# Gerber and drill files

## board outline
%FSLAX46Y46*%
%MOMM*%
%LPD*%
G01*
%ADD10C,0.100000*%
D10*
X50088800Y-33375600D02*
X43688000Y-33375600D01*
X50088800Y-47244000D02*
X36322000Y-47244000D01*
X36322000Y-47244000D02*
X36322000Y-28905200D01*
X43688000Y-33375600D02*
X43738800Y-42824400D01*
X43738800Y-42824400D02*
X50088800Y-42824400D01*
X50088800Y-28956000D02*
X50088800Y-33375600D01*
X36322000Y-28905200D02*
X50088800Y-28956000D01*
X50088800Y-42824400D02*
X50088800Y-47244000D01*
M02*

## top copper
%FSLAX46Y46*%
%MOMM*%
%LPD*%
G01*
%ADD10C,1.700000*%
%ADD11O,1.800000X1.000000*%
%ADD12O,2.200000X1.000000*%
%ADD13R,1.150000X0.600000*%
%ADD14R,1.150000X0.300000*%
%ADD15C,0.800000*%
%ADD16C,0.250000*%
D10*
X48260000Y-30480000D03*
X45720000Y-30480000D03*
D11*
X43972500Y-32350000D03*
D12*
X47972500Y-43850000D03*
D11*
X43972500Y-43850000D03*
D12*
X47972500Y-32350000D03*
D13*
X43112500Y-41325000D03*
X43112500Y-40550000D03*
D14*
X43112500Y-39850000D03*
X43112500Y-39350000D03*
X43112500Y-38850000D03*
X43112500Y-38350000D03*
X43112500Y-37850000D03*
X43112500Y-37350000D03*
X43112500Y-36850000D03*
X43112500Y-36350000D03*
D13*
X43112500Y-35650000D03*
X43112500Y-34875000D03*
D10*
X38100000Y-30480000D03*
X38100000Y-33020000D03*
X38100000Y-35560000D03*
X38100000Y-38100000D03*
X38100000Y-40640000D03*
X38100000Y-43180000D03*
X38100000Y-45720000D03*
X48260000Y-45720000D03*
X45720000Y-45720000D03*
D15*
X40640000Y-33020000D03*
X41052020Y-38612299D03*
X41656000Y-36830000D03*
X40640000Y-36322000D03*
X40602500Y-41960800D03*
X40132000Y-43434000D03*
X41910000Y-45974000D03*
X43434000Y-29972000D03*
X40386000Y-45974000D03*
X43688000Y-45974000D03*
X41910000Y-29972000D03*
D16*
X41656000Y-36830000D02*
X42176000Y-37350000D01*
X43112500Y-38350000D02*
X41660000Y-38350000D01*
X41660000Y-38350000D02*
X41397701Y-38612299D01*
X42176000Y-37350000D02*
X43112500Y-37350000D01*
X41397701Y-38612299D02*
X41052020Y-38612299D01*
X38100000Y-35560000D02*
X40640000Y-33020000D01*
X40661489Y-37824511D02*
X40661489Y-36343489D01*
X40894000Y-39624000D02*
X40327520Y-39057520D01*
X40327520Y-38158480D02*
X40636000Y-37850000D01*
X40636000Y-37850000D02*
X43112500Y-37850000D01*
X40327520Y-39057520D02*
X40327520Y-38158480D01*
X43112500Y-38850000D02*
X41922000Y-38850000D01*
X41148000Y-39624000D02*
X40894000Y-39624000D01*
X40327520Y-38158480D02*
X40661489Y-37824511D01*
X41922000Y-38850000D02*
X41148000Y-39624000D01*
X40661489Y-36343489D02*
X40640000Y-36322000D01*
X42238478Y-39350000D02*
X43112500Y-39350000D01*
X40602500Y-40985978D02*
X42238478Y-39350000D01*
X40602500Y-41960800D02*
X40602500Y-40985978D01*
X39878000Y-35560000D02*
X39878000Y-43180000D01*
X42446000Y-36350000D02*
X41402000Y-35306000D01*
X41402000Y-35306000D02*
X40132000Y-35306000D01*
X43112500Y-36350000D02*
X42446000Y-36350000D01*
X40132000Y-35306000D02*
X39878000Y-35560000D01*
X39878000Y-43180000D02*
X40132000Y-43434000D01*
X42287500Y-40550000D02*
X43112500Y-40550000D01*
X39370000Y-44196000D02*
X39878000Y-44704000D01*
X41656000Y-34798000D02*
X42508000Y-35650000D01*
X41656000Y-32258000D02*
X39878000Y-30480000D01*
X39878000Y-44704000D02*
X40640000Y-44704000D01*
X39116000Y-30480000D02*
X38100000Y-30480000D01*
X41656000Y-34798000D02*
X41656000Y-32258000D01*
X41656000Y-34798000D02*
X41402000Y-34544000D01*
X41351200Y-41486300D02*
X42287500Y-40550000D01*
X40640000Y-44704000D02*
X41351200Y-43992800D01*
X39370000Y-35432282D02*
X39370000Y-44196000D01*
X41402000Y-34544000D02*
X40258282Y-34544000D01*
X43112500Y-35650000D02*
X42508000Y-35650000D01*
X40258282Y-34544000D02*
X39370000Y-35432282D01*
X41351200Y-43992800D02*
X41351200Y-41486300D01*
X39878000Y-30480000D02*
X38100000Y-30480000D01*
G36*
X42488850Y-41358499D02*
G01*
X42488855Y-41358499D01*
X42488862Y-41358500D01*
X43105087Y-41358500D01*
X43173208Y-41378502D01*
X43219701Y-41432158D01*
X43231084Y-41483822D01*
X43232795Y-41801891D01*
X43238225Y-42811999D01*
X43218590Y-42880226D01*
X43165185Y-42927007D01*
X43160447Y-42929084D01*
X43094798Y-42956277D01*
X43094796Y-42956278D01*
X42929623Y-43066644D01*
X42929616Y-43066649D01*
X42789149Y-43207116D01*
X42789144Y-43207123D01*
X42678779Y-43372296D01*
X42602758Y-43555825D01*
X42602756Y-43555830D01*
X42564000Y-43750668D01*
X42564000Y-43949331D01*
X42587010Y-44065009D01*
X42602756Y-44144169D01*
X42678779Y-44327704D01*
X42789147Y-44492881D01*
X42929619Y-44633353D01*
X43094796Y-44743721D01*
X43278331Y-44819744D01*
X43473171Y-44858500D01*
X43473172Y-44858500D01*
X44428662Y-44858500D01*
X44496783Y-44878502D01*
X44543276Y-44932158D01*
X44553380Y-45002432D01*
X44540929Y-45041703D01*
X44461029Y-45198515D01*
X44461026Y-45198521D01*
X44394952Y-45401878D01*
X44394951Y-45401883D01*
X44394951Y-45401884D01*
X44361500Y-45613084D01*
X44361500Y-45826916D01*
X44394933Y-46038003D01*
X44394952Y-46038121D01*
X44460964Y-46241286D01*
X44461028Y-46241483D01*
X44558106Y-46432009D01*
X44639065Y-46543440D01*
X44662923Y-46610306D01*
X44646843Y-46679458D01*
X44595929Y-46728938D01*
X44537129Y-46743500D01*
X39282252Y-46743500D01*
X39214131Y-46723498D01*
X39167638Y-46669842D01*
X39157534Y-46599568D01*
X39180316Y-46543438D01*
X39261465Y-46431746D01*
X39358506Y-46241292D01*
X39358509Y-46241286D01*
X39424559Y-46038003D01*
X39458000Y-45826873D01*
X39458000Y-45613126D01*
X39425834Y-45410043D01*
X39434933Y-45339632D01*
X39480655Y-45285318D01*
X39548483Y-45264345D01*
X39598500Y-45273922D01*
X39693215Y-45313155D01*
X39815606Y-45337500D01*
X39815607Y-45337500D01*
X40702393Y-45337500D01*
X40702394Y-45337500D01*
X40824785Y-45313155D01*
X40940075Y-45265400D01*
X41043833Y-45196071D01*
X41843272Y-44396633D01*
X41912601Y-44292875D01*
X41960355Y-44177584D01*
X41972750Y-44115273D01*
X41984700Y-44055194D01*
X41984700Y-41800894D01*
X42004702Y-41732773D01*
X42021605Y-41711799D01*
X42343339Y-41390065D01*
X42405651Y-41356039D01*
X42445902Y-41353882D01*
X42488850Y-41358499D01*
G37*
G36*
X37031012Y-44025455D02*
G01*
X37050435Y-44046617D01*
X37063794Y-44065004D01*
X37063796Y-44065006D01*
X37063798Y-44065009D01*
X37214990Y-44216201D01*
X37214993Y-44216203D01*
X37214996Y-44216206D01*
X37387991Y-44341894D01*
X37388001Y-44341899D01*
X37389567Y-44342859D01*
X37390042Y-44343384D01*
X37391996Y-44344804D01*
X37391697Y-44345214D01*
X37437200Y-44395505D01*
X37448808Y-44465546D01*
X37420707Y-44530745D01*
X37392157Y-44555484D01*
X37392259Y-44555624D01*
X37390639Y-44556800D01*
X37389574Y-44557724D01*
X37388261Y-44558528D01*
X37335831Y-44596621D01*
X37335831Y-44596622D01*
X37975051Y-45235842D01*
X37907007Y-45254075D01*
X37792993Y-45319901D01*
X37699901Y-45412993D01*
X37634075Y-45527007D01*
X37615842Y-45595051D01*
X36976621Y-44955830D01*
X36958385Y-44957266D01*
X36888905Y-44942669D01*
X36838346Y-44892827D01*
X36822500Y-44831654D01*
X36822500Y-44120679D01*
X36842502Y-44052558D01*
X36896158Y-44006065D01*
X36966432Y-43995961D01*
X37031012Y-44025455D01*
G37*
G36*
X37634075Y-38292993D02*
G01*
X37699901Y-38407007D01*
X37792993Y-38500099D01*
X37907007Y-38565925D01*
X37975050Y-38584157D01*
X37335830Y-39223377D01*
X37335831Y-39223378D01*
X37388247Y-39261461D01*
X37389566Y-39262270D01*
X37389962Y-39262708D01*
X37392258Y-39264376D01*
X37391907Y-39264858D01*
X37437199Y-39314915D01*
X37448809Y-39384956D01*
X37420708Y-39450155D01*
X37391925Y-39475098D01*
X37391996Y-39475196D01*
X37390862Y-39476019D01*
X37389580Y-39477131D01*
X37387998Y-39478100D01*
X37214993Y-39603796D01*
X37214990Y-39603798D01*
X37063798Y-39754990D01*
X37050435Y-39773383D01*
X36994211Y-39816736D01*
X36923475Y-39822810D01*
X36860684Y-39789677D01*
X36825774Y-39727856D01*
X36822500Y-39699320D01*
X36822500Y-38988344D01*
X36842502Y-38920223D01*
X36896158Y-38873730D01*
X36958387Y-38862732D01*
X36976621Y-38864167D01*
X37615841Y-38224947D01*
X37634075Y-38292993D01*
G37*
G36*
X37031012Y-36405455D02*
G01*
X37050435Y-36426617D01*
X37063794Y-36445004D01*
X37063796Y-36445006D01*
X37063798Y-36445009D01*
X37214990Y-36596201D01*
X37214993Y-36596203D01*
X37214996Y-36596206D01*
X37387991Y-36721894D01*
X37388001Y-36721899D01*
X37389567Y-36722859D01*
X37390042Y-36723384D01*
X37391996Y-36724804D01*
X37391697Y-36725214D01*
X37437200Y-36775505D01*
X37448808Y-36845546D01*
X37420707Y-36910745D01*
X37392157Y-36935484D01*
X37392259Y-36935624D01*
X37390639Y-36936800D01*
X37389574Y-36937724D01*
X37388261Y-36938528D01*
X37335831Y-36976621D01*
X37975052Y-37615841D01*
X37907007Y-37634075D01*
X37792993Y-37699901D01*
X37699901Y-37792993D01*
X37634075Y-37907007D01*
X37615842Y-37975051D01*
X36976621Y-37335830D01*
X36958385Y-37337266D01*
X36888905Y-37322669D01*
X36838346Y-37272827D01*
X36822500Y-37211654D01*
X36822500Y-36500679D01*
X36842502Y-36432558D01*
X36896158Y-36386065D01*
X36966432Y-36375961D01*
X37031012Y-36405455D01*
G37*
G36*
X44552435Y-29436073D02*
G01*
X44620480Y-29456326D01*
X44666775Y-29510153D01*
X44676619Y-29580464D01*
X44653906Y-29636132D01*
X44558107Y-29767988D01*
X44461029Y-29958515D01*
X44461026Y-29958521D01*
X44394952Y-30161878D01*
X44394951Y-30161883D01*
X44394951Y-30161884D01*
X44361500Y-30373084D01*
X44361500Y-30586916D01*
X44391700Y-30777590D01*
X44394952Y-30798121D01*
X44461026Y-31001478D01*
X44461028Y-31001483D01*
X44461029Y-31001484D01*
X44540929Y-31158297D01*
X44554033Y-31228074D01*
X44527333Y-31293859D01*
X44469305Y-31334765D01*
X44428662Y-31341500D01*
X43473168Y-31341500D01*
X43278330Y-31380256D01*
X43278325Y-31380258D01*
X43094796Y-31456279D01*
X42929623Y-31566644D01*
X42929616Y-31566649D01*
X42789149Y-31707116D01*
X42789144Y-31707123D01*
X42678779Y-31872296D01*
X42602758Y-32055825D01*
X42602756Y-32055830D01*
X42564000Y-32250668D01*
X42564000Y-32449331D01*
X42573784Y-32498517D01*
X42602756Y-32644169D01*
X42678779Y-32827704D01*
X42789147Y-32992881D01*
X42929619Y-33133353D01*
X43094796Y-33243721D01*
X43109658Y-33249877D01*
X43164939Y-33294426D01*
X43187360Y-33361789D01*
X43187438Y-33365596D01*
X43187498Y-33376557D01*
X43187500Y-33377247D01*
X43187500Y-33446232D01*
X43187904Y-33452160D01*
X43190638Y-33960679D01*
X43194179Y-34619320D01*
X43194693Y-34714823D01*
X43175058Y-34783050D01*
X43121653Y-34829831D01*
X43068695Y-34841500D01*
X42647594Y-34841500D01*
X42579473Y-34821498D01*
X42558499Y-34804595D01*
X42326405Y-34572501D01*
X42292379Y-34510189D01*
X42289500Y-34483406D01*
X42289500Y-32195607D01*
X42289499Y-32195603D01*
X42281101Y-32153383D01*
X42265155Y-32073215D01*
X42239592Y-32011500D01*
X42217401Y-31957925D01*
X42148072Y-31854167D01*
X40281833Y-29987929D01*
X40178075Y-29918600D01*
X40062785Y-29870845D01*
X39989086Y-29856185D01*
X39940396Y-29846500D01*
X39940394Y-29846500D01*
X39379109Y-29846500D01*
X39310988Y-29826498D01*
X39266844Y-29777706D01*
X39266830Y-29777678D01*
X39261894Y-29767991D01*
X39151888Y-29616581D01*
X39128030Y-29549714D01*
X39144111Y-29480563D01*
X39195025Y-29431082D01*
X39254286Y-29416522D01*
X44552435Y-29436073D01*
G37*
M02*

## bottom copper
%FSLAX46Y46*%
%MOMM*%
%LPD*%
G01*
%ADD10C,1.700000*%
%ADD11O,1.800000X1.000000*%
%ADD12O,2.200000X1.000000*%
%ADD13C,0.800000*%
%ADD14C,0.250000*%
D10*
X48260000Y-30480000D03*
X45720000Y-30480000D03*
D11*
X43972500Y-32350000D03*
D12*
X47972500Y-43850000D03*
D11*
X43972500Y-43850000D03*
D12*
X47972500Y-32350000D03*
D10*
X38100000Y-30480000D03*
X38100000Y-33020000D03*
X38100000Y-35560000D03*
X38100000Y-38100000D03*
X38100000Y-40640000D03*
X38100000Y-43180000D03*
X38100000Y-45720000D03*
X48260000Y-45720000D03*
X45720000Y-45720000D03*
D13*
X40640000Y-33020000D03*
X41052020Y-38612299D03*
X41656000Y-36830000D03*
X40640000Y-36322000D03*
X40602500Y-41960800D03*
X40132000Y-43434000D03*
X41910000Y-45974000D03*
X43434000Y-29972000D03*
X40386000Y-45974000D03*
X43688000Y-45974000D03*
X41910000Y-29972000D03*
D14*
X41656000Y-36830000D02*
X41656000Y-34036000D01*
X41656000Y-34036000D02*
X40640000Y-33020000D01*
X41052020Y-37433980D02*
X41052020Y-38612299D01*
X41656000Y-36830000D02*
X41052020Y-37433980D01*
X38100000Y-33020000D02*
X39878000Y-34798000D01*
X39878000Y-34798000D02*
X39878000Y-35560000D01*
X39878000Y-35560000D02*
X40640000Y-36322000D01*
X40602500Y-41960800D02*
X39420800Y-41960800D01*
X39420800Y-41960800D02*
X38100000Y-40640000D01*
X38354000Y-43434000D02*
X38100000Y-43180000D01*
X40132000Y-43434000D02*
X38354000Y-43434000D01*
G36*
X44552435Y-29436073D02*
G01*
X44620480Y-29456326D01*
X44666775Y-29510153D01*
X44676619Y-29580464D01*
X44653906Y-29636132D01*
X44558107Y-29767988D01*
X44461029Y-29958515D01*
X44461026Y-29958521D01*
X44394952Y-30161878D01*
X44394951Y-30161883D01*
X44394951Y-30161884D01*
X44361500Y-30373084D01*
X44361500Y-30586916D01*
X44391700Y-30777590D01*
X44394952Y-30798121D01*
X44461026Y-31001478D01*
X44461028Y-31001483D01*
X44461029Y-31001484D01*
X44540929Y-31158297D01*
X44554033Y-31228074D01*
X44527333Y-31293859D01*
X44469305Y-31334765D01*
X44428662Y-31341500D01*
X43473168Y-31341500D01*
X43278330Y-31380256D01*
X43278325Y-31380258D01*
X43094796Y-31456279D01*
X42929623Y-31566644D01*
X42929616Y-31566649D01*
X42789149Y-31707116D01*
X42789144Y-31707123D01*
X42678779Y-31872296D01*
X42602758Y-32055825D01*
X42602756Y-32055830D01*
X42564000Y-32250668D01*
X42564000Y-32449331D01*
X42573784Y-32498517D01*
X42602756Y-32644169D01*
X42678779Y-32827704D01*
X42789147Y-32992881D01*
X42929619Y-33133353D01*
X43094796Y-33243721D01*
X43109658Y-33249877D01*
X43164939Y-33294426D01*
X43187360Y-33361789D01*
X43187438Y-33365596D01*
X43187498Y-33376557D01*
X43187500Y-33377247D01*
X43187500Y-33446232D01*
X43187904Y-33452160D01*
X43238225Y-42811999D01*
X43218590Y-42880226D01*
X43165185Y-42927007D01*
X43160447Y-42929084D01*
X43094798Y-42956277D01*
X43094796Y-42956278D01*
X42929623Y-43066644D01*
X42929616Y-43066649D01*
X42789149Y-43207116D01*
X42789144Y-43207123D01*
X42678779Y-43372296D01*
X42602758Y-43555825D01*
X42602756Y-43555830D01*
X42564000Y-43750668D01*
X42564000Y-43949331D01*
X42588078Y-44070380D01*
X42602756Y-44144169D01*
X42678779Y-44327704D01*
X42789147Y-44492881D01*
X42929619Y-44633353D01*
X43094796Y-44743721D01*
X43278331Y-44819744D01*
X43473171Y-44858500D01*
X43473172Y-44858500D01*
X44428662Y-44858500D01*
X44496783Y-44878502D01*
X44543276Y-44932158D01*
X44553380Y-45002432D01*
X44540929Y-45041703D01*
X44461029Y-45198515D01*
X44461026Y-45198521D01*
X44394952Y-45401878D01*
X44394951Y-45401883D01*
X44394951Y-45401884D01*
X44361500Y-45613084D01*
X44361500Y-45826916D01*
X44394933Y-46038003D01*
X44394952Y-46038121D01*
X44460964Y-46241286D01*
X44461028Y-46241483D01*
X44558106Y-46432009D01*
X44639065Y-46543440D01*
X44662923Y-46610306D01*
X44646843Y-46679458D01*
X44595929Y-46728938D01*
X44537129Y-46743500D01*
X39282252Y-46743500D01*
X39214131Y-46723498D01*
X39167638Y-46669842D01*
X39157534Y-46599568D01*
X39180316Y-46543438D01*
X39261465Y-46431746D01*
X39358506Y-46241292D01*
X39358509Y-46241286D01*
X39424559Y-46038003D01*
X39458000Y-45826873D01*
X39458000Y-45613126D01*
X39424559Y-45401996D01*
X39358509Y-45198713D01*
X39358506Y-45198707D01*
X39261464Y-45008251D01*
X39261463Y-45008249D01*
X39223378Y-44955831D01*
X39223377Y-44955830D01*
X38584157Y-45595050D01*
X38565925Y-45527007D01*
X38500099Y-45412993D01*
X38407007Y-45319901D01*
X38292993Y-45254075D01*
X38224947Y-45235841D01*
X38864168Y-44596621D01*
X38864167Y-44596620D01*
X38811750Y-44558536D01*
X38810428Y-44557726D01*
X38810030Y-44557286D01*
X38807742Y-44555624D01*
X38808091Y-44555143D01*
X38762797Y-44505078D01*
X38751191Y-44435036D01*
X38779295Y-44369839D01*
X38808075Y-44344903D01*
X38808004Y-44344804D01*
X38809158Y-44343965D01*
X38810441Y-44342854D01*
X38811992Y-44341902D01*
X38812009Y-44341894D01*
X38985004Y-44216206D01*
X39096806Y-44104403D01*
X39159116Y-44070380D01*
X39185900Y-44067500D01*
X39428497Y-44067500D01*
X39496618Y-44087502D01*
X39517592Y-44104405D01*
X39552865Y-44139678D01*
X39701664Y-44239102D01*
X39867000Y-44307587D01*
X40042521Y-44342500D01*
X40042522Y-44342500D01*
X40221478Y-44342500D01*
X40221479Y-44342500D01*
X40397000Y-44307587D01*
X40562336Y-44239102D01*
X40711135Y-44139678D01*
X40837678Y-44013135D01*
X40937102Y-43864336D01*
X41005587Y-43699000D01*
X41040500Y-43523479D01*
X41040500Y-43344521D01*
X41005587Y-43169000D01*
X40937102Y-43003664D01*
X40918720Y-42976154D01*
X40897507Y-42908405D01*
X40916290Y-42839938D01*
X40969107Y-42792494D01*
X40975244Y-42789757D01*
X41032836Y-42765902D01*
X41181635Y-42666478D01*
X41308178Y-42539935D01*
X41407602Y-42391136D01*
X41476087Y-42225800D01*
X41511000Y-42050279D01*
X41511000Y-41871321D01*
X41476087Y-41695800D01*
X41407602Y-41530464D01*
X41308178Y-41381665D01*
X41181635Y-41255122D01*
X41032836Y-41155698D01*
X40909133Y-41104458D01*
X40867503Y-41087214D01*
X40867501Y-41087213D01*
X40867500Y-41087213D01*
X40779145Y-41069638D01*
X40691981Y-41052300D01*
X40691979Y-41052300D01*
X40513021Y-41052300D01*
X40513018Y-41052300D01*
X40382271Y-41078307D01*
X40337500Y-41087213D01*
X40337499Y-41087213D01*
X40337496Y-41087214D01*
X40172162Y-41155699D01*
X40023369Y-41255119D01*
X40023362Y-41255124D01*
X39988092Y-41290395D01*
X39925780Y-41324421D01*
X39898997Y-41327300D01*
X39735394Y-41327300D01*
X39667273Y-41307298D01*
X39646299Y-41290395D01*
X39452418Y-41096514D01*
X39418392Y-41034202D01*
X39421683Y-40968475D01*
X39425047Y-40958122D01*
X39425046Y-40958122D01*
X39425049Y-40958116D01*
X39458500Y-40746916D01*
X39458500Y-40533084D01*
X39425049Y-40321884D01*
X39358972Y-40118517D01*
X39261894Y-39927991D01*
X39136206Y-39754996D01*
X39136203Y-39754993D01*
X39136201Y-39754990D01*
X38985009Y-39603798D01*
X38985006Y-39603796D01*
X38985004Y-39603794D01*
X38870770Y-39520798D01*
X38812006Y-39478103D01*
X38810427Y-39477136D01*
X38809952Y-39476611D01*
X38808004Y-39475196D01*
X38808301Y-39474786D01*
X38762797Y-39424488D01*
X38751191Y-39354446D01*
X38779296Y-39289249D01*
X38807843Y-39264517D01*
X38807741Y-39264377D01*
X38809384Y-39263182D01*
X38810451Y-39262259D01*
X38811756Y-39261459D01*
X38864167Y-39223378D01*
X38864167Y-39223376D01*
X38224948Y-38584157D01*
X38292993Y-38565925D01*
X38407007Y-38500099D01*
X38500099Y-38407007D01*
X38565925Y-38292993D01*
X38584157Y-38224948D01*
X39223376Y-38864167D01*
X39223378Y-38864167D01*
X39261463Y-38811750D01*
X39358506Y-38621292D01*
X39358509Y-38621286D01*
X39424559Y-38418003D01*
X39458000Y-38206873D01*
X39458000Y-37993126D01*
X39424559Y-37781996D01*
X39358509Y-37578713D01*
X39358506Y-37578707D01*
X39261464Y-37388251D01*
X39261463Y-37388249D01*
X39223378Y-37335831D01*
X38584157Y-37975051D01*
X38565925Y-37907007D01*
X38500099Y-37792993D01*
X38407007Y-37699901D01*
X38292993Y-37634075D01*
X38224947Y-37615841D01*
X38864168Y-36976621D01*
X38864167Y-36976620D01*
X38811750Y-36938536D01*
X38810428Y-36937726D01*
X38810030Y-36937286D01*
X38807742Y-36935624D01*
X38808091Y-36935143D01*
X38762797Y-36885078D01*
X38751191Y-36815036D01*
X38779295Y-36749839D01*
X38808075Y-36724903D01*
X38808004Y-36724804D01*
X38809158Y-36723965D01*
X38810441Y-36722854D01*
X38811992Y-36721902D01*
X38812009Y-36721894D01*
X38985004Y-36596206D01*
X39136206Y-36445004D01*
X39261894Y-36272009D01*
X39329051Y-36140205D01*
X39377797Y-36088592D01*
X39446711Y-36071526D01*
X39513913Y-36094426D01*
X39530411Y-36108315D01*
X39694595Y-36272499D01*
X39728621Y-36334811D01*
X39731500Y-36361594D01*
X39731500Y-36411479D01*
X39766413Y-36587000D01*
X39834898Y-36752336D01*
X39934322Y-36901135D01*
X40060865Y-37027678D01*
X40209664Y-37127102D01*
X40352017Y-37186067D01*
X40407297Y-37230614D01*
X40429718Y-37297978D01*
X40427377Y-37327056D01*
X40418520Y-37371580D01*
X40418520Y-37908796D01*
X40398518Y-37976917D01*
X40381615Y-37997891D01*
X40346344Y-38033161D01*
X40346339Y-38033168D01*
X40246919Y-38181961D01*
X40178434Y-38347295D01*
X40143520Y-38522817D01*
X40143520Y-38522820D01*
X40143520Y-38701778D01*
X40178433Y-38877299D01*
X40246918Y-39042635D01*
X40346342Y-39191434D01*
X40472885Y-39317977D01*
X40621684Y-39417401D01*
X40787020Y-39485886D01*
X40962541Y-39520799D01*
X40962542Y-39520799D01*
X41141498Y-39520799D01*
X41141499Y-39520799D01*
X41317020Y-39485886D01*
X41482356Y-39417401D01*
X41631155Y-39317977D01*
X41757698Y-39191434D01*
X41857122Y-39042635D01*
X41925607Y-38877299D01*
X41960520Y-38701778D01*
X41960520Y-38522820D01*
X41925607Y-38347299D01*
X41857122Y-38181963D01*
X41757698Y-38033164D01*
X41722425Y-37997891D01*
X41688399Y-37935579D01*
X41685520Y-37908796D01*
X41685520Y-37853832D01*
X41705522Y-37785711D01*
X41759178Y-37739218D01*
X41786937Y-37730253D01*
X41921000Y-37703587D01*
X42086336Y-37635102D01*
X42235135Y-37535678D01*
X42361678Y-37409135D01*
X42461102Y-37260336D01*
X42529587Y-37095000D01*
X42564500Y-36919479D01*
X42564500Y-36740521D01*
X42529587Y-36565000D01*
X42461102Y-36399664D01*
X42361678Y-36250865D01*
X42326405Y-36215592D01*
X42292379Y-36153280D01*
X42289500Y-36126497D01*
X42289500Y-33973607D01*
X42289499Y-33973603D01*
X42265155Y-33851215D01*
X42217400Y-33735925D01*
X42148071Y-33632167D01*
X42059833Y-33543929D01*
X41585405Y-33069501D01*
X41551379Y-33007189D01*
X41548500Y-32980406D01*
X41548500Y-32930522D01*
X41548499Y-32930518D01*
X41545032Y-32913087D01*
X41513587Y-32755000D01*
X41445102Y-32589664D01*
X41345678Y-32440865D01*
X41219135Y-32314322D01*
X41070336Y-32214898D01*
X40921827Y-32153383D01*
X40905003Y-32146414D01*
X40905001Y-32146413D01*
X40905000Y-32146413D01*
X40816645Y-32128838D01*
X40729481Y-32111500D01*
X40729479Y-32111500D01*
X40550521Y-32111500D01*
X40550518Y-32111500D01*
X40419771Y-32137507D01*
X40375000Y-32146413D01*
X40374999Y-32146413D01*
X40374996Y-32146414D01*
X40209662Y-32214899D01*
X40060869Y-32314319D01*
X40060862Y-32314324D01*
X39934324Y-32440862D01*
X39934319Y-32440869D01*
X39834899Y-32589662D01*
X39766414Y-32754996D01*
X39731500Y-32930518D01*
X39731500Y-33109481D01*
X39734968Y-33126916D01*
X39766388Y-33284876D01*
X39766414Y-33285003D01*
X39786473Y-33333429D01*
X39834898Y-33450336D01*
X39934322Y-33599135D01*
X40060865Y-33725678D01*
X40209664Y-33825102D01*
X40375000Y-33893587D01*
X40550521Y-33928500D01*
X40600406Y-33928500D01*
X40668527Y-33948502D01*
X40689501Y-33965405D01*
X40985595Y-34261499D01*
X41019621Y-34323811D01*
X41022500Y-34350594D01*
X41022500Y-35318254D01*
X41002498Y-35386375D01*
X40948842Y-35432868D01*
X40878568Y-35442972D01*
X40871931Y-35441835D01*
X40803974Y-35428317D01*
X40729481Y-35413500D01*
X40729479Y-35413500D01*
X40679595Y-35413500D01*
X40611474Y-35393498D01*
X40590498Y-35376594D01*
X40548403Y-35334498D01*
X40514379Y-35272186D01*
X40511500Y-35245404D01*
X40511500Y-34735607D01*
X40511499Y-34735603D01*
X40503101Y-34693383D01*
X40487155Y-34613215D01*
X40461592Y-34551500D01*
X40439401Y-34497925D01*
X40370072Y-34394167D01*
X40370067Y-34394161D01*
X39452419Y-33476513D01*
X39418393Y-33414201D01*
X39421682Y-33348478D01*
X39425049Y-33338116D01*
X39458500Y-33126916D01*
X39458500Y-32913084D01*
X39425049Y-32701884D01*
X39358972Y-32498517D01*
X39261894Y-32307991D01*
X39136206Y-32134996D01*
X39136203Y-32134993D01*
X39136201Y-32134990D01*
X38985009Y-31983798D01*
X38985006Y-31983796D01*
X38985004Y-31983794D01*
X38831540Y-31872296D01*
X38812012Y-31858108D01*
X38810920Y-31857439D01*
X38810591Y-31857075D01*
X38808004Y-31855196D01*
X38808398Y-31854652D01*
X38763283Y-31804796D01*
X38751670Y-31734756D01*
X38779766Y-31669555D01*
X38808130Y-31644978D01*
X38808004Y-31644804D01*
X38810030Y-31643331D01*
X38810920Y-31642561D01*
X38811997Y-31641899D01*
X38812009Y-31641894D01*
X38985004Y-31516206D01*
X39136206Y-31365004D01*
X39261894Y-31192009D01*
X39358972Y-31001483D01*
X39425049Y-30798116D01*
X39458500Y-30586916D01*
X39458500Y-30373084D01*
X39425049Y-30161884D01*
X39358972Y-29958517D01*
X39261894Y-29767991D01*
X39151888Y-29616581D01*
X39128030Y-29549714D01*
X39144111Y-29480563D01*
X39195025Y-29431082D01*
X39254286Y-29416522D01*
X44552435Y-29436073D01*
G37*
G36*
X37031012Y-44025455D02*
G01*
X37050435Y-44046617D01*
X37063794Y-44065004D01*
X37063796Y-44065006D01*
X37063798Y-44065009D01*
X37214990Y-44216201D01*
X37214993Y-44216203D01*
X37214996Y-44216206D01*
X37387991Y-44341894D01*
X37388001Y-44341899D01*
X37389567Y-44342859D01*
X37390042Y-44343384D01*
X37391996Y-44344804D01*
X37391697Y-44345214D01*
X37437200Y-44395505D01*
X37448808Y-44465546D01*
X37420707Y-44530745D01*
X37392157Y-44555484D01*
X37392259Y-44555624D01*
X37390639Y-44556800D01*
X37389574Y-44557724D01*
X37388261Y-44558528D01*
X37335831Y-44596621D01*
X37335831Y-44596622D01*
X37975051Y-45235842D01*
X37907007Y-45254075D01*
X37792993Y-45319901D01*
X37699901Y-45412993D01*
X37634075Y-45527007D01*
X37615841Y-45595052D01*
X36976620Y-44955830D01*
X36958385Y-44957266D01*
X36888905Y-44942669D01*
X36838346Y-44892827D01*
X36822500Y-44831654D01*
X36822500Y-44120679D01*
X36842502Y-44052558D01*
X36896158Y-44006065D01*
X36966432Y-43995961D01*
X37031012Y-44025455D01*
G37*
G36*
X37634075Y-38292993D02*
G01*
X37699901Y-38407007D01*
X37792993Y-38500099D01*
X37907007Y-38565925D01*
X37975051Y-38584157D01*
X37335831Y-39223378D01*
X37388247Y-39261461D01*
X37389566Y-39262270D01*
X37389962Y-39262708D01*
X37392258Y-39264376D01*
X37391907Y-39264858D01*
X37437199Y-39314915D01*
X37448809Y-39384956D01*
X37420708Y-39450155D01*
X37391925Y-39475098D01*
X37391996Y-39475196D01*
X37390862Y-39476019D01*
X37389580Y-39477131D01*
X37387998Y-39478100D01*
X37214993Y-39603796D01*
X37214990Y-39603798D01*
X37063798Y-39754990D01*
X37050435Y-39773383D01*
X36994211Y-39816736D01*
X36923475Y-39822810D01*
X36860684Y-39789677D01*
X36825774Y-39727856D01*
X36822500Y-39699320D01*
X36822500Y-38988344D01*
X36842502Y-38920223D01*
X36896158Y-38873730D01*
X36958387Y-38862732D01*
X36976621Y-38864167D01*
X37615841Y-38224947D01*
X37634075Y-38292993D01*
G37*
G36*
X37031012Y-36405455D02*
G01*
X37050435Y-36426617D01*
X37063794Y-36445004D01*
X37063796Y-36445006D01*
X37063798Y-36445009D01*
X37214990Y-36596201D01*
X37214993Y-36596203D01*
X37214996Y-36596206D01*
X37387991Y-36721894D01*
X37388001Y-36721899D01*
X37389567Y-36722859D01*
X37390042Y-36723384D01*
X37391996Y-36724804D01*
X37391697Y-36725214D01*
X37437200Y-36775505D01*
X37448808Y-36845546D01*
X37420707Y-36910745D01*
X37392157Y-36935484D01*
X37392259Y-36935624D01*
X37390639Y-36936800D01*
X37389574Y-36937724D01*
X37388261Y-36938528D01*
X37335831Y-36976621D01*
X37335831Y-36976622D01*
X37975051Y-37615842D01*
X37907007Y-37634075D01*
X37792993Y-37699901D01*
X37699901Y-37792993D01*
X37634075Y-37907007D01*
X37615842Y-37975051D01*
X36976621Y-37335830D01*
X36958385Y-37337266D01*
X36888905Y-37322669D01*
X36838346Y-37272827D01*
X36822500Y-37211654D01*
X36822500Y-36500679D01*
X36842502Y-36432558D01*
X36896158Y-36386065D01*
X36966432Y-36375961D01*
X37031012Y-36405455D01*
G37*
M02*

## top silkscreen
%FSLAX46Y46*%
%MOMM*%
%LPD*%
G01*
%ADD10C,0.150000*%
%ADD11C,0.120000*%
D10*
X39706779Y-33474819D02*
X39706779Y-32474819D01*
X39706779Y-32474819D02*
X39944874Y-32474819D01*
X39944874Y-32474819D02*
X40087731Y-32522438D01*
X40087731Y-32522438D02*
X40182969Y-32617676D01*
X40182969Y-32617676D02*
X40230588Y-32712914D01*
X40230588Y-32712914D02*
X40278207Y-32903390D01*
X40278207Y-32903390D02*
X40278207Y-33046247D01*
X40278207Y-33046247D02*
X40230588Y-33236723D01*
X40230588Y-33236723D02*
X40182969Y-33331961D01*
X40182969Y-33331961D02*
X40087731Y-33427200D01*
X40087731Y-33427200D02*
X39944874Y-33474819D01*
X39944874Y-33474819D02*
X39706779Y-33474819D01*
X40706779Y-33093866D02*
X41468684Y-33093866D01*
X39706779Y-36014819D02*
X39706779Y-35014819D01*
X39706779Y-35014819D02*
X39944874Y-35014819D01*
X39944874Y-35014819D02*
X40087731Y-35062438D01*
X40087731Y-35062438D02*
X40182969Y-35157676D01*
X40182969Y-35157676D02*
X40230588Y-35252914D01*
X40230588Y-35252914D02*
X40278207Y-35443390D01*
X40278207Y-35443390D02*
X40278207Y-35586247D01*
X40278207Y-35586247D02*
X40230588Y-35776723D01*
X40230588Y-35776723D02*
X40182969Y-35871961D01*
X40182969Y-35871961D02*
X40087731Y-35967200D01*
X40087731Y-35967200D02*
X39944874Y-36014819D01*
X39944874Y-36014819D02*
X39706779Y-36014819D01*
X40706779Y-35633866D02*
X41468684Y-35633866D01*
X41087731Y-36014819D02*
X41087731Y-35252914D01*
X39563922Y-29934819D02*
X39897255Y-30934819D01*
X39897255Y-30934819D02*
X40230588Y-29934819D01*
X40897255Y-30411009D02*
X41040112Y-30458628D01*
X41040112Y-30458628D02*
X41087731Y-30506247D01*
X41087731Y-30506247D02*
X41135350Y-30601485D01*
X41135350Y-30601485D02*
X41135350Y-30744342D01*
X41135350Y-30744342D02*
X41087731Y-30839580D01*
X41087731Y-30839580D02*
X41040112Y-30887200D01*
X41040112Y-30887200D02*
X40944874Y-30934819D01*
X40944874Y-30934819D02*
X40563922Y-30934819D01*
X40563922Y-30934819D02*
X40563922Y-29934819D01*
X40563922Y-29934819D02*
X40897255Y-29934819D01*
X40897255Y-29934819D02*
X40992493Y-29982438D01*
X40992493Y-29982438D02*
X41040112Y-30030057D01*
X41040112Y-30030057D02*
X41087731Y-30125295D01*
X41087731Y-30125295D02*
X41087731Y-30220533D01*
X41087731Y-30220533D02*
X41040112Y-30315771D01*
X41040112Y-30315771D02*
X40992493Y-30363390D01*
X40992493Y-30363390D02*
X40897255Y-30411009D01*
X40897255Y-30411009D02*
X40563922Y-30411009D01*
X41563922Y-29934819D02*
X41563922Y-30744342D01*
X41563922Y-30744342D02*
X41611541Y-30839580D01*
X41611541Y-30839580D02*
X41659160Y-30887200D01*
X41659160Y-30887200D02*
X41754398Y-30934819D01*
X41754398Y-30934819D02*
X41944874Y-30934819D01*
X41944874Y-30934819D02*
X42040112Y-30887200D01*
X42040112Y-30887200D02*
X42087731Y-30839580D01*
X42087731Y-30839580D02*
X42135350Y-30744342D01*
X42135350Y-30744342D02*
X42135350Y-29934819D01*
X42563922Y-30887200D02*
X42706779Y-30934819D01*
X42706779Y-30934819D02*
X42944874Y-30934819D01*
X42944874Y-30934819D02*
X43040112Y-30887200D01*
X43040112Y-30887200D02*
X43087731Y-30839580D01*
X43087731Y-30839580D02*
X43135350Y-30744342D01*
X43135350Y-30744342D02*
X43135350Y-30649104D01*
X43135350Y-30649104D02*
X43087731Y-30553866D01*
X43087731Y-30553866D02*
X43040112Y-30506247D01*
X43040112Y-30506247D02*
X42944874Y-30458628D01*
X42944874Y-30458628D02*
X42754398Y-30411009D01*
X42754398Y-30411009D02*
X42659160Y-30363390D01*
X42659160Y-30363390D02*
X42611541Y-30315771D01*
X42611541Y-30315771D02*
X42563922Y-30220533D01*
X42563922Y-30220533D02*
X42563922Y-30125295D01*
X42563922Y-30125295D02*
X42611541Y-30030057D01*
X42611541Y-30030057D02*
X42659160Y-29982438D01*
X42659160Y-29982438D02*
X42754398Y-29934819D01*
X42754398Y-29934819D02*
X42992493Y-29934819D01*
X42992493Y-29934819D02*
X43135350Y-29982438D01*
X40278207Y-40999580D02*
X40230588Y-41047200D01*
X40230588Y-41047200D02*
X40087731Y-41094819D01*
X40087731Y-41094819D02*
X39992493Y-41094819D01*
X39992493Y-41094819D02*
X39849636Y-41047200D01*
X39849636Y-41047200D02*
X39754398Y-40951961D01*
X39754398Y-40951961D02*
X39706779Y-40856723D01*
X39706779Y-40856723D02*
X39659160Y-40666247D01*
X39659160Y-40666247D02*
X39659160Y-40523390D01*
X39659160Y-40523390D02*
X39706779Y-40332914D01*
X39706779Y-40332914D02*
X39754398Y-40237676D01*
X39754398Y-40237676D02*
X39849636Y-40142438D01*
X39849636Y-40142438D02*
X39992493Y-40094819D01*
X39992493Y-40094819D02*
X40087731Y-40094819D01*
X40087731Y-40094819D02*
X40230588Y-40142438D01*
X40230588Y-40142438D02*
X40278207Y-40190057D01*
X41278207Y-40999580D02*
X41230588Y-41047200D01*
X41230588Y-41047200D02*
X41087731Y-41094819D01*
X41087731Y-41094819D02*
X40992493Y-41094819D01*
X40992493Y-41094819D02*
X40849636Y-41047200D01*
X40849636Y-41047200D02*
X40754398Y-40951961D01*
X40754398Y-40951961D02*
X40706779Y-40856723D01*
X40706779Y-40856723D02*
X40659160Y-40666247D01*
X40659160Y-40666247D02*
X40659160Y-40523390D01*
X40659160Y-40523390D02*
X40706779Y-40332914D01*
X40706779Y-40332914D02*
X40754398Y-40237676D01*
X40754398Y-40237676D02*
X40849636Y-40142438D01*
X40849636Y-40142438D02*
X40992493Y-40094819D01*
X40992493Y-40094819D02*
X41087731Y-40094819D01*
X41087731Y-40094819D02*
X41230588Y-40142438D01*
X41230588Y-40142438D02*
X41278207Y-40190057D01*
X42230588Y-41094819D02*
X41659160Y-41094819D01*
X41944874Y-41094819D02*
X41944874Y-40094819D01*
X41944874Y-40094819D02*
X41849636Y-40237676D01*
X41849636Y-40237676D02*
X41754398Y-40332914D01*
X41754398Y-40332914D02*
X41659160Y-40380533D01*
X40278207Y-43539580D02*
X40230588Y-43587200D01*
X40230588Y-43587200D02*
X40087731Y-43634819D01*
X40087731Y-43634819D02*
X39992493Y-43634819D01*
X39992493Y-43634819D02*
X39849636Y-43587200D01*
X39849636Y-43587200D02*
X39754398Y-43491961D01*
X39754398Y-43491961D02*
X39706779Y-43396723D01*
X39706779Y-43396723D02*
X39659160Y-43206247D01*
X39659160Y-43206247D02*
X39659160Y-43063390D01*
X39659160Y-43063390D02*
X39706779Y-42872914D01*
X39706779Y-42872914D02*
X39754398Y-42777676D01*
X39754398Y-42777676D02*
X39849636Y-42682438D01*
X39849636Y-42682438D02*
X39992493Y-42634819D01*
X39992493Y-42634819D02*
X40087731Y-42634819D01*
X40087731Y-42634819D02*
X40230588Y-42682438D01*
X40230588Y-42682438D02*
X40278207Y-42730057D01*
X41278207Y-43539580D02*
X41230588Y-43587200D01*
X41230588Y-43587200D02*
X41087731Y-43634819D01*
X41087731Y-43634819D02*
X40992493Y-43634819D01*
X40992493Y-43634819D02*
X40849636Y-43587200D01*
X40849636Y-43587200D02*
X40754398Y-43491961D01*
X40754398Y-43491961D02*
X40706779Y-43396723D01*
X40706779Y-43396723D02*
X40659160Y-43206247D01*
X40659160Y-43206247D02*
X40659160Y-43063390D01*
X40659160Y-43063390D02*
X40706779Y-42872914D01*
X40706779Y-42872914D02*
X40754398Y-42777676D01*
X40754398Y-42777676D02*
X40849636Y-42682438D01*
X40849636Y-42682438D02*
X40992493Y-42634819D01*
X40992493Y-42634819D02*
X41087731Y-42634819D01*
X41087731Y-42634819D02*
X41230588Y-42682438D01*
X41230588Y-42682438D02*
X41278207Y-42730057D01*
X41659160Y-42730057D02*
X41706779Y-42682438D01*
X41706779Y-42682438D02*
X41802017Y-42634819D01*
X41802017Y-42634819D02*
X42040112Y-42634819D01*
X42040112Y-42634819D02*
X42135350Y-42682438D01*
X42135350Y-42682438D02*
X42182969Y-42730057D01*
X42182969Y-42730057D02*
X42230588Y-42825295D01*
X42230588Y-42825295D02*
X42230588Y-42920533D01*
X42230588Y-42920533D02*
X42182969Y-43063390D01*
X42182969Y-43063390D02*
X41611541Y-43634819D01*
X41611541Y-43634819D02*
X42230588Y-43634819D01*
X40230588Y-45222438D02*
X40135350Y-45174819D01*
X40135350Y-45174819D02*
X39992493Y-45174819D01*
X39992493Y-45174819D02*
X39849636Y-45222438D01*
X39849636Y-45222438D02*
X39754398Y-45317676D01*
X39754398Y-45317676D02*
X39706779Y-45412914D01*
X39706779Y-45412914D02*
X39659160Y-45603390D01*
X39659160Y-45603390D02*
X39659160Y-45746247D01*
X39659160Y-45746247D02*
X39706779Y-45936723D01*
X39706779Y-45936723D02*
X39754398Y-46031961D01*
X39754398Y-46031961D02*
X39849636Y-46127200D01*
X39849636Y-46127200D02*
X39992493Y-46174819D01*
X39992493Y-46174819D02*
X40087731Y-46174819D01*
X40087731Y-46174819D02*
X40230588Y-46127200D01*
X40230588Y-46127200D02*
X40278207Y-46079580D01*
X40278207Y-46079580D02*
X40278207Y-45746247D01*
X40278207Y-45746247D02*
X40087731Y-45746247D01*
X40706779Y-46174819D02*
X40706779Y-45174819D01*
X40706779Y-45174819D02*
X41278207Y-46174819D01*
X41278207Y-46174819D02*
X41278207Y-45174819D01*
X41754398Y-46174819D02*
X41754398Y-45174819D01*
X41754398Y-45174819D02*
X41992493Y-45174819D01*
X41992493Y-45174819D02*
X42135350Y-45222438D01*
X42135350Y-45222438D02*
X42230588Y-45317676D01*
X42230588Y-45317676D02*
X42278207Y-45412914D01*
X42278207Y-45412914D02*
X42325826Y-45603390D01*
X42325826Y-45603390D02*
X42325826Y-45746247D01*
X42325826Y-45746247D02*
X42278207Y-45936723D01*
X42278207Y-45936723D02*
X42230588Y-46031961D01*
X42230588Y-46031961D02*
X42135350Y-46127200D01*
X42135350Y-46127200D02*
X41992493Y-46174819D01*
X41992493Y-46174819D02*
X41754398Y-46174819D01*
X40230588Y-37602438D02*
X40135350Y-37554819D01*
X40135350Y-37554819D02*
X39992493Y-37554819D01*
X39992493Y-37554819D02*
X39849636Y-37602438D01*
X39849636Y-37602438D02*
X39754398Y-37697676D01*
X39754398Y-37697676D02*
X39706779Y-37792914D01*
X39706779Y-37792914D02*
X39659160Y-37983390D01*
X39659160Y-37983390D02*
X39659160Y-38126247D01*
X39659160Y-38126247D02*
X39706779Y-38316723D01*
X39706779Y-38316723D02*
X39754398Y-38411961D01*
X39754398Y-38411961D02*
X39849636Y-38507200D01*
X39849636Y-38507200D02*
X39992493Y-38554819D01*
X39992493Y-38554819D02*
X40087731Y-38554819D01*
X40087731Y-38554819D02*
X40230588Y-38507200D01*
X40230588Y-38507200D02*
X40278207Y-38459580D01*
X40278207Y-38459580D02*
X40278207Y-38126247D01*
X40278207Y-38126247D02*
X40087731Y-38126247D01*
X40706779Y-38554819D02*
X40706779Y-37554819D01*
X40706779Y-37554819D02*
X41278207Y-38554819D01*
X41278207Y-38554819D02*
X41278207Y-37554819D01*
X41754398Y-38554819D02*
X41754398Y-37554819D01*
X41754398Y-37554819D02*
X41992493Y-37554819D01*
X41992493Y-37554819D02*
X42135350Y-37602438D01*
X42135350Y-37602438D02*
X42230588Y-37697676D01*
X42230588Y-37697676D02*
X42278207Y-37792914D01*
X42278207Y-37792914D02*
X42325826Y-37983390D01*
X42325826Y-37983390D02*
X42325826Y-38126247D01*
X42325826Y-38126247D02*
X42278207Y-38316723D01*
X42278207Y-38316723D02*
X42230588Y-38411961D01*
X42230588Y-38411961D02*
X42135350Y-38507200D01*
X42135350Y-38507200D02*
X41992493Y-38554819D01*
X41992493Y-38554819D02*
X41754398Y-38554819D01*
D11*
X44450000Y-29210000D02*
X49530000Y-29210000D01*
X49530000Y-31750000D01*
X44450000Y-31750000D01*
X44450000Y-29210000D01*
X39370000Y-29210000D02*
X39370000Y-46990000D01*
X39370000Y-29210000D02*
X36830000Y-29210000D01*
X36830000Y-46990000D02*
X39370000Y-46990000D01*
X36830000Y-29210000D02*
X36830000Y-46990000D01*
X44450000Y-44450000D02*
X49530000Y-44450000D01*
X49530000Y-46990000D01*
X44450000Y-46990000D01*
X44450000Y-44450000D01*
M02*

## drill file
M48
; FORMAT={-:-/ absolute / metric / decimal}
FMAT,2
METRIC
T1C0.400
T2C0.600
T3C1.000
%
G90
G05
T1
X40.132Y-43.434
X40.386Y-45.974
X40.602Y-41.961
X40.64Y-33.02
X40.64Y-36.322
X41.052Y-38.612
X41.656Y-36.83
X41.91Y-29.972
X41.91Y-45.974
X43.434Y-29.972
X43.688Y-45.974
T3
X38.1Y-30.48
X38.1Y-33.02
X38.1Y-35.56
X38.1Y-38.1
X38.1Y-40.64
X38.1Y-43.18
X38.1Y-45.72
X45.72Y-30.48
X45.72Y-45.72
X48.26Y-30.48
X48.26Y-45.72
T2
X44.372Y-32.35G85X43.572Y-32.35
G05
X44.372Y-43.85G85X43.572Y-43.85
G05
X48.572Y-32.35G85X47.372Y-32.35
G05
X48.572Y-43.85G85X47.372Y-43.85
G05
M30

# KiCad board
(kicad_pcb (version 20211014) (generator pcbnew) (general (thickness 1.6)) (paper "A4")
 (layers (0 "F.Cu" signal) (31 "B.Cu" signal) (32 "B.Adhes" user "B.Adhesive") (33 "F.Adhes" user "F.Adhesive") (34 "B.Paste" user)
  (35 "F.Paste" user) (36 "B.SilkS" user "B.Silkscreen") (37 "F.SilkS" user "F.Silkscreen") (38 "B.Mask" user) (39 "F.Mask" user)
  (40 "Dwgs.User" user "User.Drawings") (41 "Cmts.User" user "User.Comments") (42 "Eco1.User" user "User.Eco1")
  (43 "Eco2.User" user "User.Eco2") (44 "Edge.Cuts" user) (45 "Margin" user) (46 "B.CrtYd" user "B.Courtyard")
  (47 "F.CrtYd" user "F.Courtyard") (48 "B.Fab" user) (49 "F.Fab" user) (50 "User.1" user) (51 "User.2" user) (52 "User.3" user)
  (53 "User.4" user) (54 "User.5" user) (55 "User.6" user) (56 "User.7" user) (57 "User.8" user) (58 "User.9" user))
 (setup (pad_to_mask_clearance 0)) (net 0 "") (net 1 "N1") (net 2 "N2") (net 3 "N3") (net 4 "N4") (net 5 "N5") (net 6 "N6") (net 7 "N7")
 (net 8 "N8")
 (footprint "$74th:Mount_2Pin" (layer "F.Cu") (at 46.99 30.48 90)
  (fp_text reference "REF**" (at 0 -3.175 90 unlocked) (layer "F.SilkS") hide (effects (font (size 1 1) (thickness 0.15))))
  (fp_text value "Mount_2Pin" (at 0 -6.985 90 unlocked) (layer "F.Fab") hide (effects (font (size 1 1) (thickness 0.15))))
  (fp_rect (start -1.27 -2.54) (end 1.27 2.54) (layer "F.SilkS") (width 0.12) (fill none))
  (pad "" thru_hole circle (at 0 1.27) (size 1.7 1.7) (drill 1) (layers *.Cu *.Mask))
  (pad "" thru_hole circle (at 0 -1.27) (size 1.7 1.7) (drill 1) (layers *.Cu *.Mask)))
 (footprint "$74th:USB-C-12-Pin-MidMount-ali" (layer "F.Cu") (at 43.1125 38.1 90)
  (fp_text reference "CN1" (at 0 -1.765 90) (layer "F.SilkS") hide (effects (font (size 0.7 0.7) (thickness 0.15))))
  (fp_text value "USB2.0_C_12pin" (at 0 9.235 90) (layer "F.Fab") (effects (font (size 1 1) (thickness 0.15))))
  (pad "" thru_hole oval (at 5.75 0.86 270) (size 1 1.8) (drill oval 0.6 1.4) (layers *.Cu *.Mask))
  (pad "" thru_hole oval (at -5.75 4.86 270) (size 1 2.2) (drill oval 0.6 1.8) (layers *.Cu *.Mask))
  (pad "" thru_hole oval (at -5.75 0.86 270) (size 1 1.8) (drill oval 0.6 1.4) (layers *.Cu *.Mask))
  (pad "" thru_hole oval (at 5.75 4.86 270) (size 1 2.2) (drill oval 0.6 1.8) (layers *.Cu *.Mask))
  (pad "1" smd rect (at -3.225 0 270) (size 0.6 1.15) (layers "F.Cu" "F.Paste" "F.Mask") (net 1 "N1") (zone_connect 2))
  (pad "2" smd rect (at -2.45 0 270) (size 0.6 1.15) (layers "F.Cu" "F.Paste" "F.Mask") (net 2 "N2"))
  (pad "3" smd rect (at -1.75 0 270) (size 0.3 1.15) (layers "F.Cu" "F.Paste" "F.Mask") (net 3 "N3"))
  (pad "4" smd rect (at -1.25 0 270) (size 0.3 1.15) (layers "F.Cu" "F.Paste" "F.Mask") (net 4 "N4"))
  (pad "5" smd rect (at -0.75 0 270) (size 0.3 1.15) (layers "F.Cu" "F.Paste" "F.Mask") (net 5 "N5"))
  (pad "6" smd rect (at -0.25 0 270) (size 0.3 1.15) (layers "F.Cu" "F.Paste" "F.Mask") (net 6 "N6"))
  (pad "7" smd rect (at 0.25 0 270) (size 0.3 1.15) (layers "F.Cu" "F.Paste" "F.Mask") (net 5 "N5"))
  (pad "8" smd rect (at 0.75 0 270) (size 0.3 1.15) (layers "F.Cu" "F.Paste" "F.Mask") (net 6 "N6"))
  (pad "9" smd rect (at 1.25 0 270) (size 0.3 1.15) (layers "F.Cu" "F.Paste" "F.Mask") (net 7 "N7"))
  (pad "10" smd rect (at 1.75 0 270) (size 0.3 1.15) (layers "F.Cu" "F.Paste" "F.Mask") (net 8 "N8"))
  (pad "11" smd rect (at 2.45 0 270) (size 0.6 1.15) (layers "F.Cu" "F.Paste" "F.Mask") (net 2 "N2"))
  (pad "12" smd rect (at 3.225 0 270) (size 0.6 1.15) (layers "F.Cu" "F.Paste" "F.Mask") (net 1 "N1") (zone_connect 2)))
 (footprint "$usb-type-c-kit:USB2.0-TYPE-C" (layer "F.Cu") (at 38.1 38.1)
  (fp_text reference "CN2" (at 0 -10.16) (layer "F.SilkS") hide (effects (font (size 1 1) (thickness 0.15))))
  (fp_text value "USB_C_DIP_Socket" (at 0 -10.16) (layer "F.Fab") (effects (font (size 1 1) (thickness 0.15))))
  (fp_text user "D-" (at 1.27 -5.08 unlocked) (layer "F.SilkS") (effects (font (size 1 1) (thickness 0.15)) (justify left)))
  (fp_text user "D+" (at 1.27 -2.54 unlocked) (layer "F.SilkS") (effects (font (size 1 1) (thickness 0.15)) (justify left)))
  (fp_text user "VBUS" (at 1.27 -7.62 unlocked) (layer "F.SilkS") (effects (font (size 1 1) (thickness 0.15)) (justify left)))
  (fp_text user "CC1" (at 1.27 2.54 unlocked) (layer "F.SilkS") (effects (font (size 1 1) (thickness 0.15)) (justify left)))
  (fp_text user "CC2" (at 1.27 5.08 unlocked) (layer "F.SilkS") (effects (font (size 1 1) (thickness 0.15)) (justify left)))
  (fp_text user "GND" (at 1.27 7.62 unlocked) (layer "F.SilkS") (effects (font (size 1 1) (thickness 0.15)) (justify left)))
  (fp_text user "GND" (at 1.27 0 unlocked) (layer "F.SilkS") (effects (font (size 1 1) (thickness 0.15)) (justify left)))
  (fp_line (start 1.27 -8.89) (end 1.27 8.89) (layer "F.SilkS") (width 0.12))
  (fp_line (start 1.27 -8.89) (end -1.27 -8.89) (layer "F.SilkS") (width 0.12))
  (fp_line (start -1.27 8.89) (end 1.27 8.89) (layer "F.SilkS") (width 0.12))
  (fp_line (start -1.27 -8.89) (end -1.27 8.89) (layer "F.SilkS") (width 0.12))
  (pad "1" thru_hole circle (at 0 -7.62 270) (size 1.7 1.7) (drill 1) (layers *.Cu *.Mask) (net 2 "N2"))
  (pad "2" thru_hole circle (at 0 -5.08 270) (size 1.7 1.7) (drill 1) (layers *.Cu *.Mask) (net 5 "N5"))
  (pad "3" thru_hole circle (at 0 -2.54 270) (size 1.7 1.7) (drill 1) (layers *.Cu *.Mask) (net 6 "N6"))
  (pad "4" thru_hole circle (at 0 0 270) (size 1.7 1.7) (drill 1) (layers *.Cu *.Mask) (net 1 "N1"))
  (pad "5" thru_hole circle (at 0 2.54 270) (size 1.7 1.7) (drill 1) (layers *.Cu *.Mask) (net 4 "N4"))
  (pad "6" thru_hole circle (at 0 5.08 270) (size 1.7 1.7) (drill 1) (layers *.Cu *.Mask) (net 8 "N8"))
  (pad "7" thru_hole circle (at 0 7.62 270) (size 1.7 1.7) (drill 1) (layers *.Cu *.Mask) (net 1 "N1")))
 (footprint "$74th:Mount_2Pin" (layer "F.Cu") (at 46.99 45.72 90)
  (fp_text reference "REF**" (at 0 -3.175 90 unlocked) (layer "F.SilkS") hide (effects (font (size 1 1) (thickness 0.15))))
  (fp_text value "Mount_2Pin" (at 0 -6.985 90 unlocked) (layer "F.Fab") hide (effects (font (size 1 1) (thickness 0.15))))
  (fp_rect (start -1.27 -2.54) (end 1.27 2.54) (layer "F.SilkS") (width 0.12) (fill none))
  (pad "" thru_hole circle (at 0 1.27) (size 1.7 1.7) (drill 1) (layers *.Cu *.Mask))
  (pad "" thru_hole circle (at 0 -1.27) (size 1.7 1.7) (drill 1) (layers *.Cu *.Mask)))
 (gr_line (start 50.0888 33.3756) (end 43.688 33.3756) (layer "Edge.Cuts") (width 0.1))
 (gr_line (start 50.0888 47.244) (end 36.322 47.244) (layer "Edge.Cuts") (width 0.1))
 (gr_line (start 36.322 47.244) (end 36.322 28.9052) (layer "Edge.Cuts") (width 0.1))
 (gr_line (start 43.688 33.3756) (end 43.7388 42.8244) (layer "Edge.Cuts") (width 0.1))
 (gr_line (start 43.7388 42.8244) (end 50.0888 42.8244) (layer "Edge.Cuts") (width 0.1))
 (gr_line (start 50.0888 28.956) (end 50.0888 33.3756) (layer "Edge.Cuts") (width 0.1))
 (gr_line (start 36.322 28.9052) (end 50.0888 28.956) (layer "Edge.Cuts") (width 0.1))
 (gr_line (start 50.0888 42.8244) (end 50.0888 47.244) (layer "Edge.Cuts") (width 0.1))
 (segment (start 41.656 36.83) (end 42.176 37.35) (width 0.25) (layer "F.Cu") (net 6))
 (segment (start 43.1125 38.35) (end 41.66 38.35) (width 0.25) (layer "F.Cu") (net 6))
 (segment (start 41.66 38.35) (end 41.397701 38.612299) (width 0.25) (layer "F.Cu") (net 6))
 (segment (start 42.176 37.35) (end 43.1125 37.35) (width 0.25) (layer "F.Cu") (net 6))
 (segment (start 41.397701 38.612299) (end 41.05202 38.612299) (width 0.25) (layer "F.Cu") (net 6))
 (segment (start 38.1 35.56) (end 40.64 33.02) (width 0.25) (layer "F.Cu") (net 6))
 (via (at 40.64 33.02) (size 0.8) (drill 0.4) (layers "F.Cu" "B.Cu") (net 6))
 (via (at 41.05202 38.612299) (size 0.8) (drill 0.4) (layers "F.Cu" "B.Cu") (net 6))
 (via (at 41.656 36.83) (size 0.8) (drill 0.4) (layers "F.Cu" "B.Cu") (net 6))
 (segment (start 41.656 36.83) (end 41.656 34.036) (width 0.25) (layer "B.Cu") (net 6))
 (segment (start 41.656 34.036) (end 40.64 33.02) (width 0.25) (layer "B.Cu") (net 6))
 (segment (start 41.05202 37.43398) (end 41.05202 38.612299) (width 0.25) (layer "B.Cu") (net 6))
 (segment (start 41.656 36.83) (end 41.05202 37.43398) (width 0.25) (layer "B.Cu") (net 6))
 (segment (start 40.661489 37.824511) (end 40.661489 36.343489) (width 0.25) (layer "F.Cu") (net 5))
 (segment (start 40.894 39.624) (end 40.32752 39.05752) (width 0.25) (layer "F.Cu") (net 5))
 (segment (start 40.32752 38.15848) (end 40.636 37.85) (width 0.25) (layer "F.Cu") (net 5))
 (segment (start 40.636 37.85) (end 43.1125 37.85) (width 0.25) (layer "F.Cu") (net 5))
 (segment (start 40.32752 39.05752) (end 40.32752 38.15848) (width 0.25) (layer "F.Cu") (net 5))
 (segment (start 43.1125 38.85) (end 41.922 38.85) (width 0.25) (layer "F.Cu") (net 5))
 (segment (start 41.148 39.624) (end 40.894 39.624) (width 0.25) (layer "F.Cu") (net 5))
 (segment (start 40.32752 38.15848) (end 40.661489 37.824511) (width 0.25) (layer "F.Cu") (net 5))
 (segment (start 41.922 38.85) (end 41.148 39.624) (width 0.25) (layer "F.Cu") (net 5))
 (segment (start 40.661489 36.343489) (end 40.64 36.322) (width 0.25) (layer "F.Cu") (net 5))
 (via (at 40.64 36.322) (size 0.8) (drill 0.4) (layers "F.Cu" "B.Cu") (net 5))
 (segment (start 38.1 33.02) (end 39.878 34.798) (width 0.25) (layer "B.Cu") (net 5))
 (segment (start 39.878 34.798) (end 39.878 35.56) (width 0.25) (layer "B.Cu") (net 5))
 (segment (start 39.878 35.56) (end 40.64 36.322) (width 0.25) (layer "B.Cu") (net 5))
 (segment (start 42.238478 39.35) (end 43.1125 39.35) (width 0.25) (layer "F.Cu") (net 4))
 (segment (start 40.6025 40.985978) (end 42.238478 39.35) (width 0.25) (layer "F.Cu") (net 4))
 (segment (start 40.6025 41.9608) (end 40.6025 40.985978) (width 0.25) (layer "F.Cu") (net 4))
 (via (at 40.6025 41.9608) (size 0.8) (drill 0.4) (layers "F.Cu" "B.Cu") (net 4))
 (segment (start 40.6025 41.9608) (end 39.4208 41.9608) (width 0.25) (layer "B.Cu") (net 4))
 (segment (start 39.4208 41.9608) (end 38.1 40.64) (width 0.25) (layer "B.Cu") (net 4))
 (segment (start 39.878 35.56) (end 39.878 43.18) (width 0.25) (layer "F.Cu") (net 8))
 (segment (start 42.446 36.35) (end 41.402 35.306) (width 0.25) (layer "F.Cu") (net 8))
 (segment (start 41.402 35.306) (end 40.132 35.306) (width 0.25) (layer "F.Cu") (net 8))
 (segment (start 43.1125 36.35) (end 42.446 36.35) (width 0.25) (layer "F.Cu") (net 8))
 (segment (start 40.132 35.306) (end 39.878 35.56) (width 0.25) (layer "F.Cu") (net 8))
 (segment (start 39.878 43.18) (end 40.132 43.434) (width 0.25) (layer "F.Cu") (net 8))
 (via (at 40.132 43.434) (size 0.8) (drill 0.4) (layers "F.Cu" "B.Cu") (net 8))
 (segment (start 38.354 43.434) (end 38.1 43.18) (width 0.25) (layer "B.Cu") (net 8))
 (segment (start 40.132 43.434) (end 38.354 43.434) (width 0.25) (layer "B.Cu") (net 8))
 (segment (start 42.2875 40.55) (end 43.1125 40.55) (width 0.25) (layer "F.Cu") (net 2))
 (segment (start 39.37 44.196) (end 39.878 44.704) (width 0.25) (layer "F.Cu") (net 2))
 (segment (start 41.656 34.798) (end 42.508 35.65) (width 0.25) (layer "F.Cu") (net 2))
 (segment (start 41.656 32.258) (end 39.878 30.48) (width 0.25) (layer "F.Cu") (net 2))
 (segment (start 39.878 44.704) (end 40.64 44.704) (width 0.25) (layer "F.Cu") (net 2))
 (segment (start 39.116 30.48) (end 38.1 30.48) (width 0.25) (layer "F.Cu") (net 2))
 (segment (start 41.656 34.798) (end 41.656 32.258) (width 0.25) (layer "F.Cu") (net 2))
 (segment (start 41.656 34.798) (end 41.402 34.544) (width 0.25) (layer "F.Cu") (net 2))
 (segment (start 41.3512 41.4863) (end 42.2875 40.55) (width 0.25) (layer "F.Cu") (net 2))
 (segment (start 40.64 44.704) (end 41.3512 43.9928) (width 0.25) (layer "F.Cu") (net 2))
 (segment (start 39.37 35.432282) (end 39.37 44.196) (width 0.25) (layer "F.Cu") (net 2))
 (segment (start 41.402 34.544) (end 40.258282 34.544) (width 0.25) (layer "F.Cu") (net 2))
 (segment (start 43.1125 35.65) (end 42.508 35.65) (width 0.25) (layer "F.Cu") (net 2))
 (segment (start 40.258282 34.544) (end 39.37 35.432282) (width 0.25) (layer "F.Cu") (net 2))
 (segment (start 41.3512 43.9928) (end 41.3512 41.4863) (width 0.25) (layer "F.Cu") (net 2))
 (segment (start 39.878 30.48) (end 38.1 30.48) (width 0.25) (layer "F.Cu") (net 2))
 (via (at 41.91 45.974) (size 0.8) (drill 0.4) (layers "F.Cu" "B.Cu") (free) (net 1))
 (via (at 43.434 29.972) (size 0.8) (drill 0.4) (layers "F.Cu" "B.Cu") (free) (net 1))
 (via (at 40.386 45.974) (size 0.8) (drill 0.4) (layers "F.Cu" "B.Cu") (free) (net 1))
 (via (at 43.688 45.974) (size 0.8) (drill 0.4) (layers "F.Cu" "B.Cu") (free) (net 1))
 (via (at 41.91 29.972) (size 0.8) (drill 0.4) (layers "F.Cu" "B.Cu") (free) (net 1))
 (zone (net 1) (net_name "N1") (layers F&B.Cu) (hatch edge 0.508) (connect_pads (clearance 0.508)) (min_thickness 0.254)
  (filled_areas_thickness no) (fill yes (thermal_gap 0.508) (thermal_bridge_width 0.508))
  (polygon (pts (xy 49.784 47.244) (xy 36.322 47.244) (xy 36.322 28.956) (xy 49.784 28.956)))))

